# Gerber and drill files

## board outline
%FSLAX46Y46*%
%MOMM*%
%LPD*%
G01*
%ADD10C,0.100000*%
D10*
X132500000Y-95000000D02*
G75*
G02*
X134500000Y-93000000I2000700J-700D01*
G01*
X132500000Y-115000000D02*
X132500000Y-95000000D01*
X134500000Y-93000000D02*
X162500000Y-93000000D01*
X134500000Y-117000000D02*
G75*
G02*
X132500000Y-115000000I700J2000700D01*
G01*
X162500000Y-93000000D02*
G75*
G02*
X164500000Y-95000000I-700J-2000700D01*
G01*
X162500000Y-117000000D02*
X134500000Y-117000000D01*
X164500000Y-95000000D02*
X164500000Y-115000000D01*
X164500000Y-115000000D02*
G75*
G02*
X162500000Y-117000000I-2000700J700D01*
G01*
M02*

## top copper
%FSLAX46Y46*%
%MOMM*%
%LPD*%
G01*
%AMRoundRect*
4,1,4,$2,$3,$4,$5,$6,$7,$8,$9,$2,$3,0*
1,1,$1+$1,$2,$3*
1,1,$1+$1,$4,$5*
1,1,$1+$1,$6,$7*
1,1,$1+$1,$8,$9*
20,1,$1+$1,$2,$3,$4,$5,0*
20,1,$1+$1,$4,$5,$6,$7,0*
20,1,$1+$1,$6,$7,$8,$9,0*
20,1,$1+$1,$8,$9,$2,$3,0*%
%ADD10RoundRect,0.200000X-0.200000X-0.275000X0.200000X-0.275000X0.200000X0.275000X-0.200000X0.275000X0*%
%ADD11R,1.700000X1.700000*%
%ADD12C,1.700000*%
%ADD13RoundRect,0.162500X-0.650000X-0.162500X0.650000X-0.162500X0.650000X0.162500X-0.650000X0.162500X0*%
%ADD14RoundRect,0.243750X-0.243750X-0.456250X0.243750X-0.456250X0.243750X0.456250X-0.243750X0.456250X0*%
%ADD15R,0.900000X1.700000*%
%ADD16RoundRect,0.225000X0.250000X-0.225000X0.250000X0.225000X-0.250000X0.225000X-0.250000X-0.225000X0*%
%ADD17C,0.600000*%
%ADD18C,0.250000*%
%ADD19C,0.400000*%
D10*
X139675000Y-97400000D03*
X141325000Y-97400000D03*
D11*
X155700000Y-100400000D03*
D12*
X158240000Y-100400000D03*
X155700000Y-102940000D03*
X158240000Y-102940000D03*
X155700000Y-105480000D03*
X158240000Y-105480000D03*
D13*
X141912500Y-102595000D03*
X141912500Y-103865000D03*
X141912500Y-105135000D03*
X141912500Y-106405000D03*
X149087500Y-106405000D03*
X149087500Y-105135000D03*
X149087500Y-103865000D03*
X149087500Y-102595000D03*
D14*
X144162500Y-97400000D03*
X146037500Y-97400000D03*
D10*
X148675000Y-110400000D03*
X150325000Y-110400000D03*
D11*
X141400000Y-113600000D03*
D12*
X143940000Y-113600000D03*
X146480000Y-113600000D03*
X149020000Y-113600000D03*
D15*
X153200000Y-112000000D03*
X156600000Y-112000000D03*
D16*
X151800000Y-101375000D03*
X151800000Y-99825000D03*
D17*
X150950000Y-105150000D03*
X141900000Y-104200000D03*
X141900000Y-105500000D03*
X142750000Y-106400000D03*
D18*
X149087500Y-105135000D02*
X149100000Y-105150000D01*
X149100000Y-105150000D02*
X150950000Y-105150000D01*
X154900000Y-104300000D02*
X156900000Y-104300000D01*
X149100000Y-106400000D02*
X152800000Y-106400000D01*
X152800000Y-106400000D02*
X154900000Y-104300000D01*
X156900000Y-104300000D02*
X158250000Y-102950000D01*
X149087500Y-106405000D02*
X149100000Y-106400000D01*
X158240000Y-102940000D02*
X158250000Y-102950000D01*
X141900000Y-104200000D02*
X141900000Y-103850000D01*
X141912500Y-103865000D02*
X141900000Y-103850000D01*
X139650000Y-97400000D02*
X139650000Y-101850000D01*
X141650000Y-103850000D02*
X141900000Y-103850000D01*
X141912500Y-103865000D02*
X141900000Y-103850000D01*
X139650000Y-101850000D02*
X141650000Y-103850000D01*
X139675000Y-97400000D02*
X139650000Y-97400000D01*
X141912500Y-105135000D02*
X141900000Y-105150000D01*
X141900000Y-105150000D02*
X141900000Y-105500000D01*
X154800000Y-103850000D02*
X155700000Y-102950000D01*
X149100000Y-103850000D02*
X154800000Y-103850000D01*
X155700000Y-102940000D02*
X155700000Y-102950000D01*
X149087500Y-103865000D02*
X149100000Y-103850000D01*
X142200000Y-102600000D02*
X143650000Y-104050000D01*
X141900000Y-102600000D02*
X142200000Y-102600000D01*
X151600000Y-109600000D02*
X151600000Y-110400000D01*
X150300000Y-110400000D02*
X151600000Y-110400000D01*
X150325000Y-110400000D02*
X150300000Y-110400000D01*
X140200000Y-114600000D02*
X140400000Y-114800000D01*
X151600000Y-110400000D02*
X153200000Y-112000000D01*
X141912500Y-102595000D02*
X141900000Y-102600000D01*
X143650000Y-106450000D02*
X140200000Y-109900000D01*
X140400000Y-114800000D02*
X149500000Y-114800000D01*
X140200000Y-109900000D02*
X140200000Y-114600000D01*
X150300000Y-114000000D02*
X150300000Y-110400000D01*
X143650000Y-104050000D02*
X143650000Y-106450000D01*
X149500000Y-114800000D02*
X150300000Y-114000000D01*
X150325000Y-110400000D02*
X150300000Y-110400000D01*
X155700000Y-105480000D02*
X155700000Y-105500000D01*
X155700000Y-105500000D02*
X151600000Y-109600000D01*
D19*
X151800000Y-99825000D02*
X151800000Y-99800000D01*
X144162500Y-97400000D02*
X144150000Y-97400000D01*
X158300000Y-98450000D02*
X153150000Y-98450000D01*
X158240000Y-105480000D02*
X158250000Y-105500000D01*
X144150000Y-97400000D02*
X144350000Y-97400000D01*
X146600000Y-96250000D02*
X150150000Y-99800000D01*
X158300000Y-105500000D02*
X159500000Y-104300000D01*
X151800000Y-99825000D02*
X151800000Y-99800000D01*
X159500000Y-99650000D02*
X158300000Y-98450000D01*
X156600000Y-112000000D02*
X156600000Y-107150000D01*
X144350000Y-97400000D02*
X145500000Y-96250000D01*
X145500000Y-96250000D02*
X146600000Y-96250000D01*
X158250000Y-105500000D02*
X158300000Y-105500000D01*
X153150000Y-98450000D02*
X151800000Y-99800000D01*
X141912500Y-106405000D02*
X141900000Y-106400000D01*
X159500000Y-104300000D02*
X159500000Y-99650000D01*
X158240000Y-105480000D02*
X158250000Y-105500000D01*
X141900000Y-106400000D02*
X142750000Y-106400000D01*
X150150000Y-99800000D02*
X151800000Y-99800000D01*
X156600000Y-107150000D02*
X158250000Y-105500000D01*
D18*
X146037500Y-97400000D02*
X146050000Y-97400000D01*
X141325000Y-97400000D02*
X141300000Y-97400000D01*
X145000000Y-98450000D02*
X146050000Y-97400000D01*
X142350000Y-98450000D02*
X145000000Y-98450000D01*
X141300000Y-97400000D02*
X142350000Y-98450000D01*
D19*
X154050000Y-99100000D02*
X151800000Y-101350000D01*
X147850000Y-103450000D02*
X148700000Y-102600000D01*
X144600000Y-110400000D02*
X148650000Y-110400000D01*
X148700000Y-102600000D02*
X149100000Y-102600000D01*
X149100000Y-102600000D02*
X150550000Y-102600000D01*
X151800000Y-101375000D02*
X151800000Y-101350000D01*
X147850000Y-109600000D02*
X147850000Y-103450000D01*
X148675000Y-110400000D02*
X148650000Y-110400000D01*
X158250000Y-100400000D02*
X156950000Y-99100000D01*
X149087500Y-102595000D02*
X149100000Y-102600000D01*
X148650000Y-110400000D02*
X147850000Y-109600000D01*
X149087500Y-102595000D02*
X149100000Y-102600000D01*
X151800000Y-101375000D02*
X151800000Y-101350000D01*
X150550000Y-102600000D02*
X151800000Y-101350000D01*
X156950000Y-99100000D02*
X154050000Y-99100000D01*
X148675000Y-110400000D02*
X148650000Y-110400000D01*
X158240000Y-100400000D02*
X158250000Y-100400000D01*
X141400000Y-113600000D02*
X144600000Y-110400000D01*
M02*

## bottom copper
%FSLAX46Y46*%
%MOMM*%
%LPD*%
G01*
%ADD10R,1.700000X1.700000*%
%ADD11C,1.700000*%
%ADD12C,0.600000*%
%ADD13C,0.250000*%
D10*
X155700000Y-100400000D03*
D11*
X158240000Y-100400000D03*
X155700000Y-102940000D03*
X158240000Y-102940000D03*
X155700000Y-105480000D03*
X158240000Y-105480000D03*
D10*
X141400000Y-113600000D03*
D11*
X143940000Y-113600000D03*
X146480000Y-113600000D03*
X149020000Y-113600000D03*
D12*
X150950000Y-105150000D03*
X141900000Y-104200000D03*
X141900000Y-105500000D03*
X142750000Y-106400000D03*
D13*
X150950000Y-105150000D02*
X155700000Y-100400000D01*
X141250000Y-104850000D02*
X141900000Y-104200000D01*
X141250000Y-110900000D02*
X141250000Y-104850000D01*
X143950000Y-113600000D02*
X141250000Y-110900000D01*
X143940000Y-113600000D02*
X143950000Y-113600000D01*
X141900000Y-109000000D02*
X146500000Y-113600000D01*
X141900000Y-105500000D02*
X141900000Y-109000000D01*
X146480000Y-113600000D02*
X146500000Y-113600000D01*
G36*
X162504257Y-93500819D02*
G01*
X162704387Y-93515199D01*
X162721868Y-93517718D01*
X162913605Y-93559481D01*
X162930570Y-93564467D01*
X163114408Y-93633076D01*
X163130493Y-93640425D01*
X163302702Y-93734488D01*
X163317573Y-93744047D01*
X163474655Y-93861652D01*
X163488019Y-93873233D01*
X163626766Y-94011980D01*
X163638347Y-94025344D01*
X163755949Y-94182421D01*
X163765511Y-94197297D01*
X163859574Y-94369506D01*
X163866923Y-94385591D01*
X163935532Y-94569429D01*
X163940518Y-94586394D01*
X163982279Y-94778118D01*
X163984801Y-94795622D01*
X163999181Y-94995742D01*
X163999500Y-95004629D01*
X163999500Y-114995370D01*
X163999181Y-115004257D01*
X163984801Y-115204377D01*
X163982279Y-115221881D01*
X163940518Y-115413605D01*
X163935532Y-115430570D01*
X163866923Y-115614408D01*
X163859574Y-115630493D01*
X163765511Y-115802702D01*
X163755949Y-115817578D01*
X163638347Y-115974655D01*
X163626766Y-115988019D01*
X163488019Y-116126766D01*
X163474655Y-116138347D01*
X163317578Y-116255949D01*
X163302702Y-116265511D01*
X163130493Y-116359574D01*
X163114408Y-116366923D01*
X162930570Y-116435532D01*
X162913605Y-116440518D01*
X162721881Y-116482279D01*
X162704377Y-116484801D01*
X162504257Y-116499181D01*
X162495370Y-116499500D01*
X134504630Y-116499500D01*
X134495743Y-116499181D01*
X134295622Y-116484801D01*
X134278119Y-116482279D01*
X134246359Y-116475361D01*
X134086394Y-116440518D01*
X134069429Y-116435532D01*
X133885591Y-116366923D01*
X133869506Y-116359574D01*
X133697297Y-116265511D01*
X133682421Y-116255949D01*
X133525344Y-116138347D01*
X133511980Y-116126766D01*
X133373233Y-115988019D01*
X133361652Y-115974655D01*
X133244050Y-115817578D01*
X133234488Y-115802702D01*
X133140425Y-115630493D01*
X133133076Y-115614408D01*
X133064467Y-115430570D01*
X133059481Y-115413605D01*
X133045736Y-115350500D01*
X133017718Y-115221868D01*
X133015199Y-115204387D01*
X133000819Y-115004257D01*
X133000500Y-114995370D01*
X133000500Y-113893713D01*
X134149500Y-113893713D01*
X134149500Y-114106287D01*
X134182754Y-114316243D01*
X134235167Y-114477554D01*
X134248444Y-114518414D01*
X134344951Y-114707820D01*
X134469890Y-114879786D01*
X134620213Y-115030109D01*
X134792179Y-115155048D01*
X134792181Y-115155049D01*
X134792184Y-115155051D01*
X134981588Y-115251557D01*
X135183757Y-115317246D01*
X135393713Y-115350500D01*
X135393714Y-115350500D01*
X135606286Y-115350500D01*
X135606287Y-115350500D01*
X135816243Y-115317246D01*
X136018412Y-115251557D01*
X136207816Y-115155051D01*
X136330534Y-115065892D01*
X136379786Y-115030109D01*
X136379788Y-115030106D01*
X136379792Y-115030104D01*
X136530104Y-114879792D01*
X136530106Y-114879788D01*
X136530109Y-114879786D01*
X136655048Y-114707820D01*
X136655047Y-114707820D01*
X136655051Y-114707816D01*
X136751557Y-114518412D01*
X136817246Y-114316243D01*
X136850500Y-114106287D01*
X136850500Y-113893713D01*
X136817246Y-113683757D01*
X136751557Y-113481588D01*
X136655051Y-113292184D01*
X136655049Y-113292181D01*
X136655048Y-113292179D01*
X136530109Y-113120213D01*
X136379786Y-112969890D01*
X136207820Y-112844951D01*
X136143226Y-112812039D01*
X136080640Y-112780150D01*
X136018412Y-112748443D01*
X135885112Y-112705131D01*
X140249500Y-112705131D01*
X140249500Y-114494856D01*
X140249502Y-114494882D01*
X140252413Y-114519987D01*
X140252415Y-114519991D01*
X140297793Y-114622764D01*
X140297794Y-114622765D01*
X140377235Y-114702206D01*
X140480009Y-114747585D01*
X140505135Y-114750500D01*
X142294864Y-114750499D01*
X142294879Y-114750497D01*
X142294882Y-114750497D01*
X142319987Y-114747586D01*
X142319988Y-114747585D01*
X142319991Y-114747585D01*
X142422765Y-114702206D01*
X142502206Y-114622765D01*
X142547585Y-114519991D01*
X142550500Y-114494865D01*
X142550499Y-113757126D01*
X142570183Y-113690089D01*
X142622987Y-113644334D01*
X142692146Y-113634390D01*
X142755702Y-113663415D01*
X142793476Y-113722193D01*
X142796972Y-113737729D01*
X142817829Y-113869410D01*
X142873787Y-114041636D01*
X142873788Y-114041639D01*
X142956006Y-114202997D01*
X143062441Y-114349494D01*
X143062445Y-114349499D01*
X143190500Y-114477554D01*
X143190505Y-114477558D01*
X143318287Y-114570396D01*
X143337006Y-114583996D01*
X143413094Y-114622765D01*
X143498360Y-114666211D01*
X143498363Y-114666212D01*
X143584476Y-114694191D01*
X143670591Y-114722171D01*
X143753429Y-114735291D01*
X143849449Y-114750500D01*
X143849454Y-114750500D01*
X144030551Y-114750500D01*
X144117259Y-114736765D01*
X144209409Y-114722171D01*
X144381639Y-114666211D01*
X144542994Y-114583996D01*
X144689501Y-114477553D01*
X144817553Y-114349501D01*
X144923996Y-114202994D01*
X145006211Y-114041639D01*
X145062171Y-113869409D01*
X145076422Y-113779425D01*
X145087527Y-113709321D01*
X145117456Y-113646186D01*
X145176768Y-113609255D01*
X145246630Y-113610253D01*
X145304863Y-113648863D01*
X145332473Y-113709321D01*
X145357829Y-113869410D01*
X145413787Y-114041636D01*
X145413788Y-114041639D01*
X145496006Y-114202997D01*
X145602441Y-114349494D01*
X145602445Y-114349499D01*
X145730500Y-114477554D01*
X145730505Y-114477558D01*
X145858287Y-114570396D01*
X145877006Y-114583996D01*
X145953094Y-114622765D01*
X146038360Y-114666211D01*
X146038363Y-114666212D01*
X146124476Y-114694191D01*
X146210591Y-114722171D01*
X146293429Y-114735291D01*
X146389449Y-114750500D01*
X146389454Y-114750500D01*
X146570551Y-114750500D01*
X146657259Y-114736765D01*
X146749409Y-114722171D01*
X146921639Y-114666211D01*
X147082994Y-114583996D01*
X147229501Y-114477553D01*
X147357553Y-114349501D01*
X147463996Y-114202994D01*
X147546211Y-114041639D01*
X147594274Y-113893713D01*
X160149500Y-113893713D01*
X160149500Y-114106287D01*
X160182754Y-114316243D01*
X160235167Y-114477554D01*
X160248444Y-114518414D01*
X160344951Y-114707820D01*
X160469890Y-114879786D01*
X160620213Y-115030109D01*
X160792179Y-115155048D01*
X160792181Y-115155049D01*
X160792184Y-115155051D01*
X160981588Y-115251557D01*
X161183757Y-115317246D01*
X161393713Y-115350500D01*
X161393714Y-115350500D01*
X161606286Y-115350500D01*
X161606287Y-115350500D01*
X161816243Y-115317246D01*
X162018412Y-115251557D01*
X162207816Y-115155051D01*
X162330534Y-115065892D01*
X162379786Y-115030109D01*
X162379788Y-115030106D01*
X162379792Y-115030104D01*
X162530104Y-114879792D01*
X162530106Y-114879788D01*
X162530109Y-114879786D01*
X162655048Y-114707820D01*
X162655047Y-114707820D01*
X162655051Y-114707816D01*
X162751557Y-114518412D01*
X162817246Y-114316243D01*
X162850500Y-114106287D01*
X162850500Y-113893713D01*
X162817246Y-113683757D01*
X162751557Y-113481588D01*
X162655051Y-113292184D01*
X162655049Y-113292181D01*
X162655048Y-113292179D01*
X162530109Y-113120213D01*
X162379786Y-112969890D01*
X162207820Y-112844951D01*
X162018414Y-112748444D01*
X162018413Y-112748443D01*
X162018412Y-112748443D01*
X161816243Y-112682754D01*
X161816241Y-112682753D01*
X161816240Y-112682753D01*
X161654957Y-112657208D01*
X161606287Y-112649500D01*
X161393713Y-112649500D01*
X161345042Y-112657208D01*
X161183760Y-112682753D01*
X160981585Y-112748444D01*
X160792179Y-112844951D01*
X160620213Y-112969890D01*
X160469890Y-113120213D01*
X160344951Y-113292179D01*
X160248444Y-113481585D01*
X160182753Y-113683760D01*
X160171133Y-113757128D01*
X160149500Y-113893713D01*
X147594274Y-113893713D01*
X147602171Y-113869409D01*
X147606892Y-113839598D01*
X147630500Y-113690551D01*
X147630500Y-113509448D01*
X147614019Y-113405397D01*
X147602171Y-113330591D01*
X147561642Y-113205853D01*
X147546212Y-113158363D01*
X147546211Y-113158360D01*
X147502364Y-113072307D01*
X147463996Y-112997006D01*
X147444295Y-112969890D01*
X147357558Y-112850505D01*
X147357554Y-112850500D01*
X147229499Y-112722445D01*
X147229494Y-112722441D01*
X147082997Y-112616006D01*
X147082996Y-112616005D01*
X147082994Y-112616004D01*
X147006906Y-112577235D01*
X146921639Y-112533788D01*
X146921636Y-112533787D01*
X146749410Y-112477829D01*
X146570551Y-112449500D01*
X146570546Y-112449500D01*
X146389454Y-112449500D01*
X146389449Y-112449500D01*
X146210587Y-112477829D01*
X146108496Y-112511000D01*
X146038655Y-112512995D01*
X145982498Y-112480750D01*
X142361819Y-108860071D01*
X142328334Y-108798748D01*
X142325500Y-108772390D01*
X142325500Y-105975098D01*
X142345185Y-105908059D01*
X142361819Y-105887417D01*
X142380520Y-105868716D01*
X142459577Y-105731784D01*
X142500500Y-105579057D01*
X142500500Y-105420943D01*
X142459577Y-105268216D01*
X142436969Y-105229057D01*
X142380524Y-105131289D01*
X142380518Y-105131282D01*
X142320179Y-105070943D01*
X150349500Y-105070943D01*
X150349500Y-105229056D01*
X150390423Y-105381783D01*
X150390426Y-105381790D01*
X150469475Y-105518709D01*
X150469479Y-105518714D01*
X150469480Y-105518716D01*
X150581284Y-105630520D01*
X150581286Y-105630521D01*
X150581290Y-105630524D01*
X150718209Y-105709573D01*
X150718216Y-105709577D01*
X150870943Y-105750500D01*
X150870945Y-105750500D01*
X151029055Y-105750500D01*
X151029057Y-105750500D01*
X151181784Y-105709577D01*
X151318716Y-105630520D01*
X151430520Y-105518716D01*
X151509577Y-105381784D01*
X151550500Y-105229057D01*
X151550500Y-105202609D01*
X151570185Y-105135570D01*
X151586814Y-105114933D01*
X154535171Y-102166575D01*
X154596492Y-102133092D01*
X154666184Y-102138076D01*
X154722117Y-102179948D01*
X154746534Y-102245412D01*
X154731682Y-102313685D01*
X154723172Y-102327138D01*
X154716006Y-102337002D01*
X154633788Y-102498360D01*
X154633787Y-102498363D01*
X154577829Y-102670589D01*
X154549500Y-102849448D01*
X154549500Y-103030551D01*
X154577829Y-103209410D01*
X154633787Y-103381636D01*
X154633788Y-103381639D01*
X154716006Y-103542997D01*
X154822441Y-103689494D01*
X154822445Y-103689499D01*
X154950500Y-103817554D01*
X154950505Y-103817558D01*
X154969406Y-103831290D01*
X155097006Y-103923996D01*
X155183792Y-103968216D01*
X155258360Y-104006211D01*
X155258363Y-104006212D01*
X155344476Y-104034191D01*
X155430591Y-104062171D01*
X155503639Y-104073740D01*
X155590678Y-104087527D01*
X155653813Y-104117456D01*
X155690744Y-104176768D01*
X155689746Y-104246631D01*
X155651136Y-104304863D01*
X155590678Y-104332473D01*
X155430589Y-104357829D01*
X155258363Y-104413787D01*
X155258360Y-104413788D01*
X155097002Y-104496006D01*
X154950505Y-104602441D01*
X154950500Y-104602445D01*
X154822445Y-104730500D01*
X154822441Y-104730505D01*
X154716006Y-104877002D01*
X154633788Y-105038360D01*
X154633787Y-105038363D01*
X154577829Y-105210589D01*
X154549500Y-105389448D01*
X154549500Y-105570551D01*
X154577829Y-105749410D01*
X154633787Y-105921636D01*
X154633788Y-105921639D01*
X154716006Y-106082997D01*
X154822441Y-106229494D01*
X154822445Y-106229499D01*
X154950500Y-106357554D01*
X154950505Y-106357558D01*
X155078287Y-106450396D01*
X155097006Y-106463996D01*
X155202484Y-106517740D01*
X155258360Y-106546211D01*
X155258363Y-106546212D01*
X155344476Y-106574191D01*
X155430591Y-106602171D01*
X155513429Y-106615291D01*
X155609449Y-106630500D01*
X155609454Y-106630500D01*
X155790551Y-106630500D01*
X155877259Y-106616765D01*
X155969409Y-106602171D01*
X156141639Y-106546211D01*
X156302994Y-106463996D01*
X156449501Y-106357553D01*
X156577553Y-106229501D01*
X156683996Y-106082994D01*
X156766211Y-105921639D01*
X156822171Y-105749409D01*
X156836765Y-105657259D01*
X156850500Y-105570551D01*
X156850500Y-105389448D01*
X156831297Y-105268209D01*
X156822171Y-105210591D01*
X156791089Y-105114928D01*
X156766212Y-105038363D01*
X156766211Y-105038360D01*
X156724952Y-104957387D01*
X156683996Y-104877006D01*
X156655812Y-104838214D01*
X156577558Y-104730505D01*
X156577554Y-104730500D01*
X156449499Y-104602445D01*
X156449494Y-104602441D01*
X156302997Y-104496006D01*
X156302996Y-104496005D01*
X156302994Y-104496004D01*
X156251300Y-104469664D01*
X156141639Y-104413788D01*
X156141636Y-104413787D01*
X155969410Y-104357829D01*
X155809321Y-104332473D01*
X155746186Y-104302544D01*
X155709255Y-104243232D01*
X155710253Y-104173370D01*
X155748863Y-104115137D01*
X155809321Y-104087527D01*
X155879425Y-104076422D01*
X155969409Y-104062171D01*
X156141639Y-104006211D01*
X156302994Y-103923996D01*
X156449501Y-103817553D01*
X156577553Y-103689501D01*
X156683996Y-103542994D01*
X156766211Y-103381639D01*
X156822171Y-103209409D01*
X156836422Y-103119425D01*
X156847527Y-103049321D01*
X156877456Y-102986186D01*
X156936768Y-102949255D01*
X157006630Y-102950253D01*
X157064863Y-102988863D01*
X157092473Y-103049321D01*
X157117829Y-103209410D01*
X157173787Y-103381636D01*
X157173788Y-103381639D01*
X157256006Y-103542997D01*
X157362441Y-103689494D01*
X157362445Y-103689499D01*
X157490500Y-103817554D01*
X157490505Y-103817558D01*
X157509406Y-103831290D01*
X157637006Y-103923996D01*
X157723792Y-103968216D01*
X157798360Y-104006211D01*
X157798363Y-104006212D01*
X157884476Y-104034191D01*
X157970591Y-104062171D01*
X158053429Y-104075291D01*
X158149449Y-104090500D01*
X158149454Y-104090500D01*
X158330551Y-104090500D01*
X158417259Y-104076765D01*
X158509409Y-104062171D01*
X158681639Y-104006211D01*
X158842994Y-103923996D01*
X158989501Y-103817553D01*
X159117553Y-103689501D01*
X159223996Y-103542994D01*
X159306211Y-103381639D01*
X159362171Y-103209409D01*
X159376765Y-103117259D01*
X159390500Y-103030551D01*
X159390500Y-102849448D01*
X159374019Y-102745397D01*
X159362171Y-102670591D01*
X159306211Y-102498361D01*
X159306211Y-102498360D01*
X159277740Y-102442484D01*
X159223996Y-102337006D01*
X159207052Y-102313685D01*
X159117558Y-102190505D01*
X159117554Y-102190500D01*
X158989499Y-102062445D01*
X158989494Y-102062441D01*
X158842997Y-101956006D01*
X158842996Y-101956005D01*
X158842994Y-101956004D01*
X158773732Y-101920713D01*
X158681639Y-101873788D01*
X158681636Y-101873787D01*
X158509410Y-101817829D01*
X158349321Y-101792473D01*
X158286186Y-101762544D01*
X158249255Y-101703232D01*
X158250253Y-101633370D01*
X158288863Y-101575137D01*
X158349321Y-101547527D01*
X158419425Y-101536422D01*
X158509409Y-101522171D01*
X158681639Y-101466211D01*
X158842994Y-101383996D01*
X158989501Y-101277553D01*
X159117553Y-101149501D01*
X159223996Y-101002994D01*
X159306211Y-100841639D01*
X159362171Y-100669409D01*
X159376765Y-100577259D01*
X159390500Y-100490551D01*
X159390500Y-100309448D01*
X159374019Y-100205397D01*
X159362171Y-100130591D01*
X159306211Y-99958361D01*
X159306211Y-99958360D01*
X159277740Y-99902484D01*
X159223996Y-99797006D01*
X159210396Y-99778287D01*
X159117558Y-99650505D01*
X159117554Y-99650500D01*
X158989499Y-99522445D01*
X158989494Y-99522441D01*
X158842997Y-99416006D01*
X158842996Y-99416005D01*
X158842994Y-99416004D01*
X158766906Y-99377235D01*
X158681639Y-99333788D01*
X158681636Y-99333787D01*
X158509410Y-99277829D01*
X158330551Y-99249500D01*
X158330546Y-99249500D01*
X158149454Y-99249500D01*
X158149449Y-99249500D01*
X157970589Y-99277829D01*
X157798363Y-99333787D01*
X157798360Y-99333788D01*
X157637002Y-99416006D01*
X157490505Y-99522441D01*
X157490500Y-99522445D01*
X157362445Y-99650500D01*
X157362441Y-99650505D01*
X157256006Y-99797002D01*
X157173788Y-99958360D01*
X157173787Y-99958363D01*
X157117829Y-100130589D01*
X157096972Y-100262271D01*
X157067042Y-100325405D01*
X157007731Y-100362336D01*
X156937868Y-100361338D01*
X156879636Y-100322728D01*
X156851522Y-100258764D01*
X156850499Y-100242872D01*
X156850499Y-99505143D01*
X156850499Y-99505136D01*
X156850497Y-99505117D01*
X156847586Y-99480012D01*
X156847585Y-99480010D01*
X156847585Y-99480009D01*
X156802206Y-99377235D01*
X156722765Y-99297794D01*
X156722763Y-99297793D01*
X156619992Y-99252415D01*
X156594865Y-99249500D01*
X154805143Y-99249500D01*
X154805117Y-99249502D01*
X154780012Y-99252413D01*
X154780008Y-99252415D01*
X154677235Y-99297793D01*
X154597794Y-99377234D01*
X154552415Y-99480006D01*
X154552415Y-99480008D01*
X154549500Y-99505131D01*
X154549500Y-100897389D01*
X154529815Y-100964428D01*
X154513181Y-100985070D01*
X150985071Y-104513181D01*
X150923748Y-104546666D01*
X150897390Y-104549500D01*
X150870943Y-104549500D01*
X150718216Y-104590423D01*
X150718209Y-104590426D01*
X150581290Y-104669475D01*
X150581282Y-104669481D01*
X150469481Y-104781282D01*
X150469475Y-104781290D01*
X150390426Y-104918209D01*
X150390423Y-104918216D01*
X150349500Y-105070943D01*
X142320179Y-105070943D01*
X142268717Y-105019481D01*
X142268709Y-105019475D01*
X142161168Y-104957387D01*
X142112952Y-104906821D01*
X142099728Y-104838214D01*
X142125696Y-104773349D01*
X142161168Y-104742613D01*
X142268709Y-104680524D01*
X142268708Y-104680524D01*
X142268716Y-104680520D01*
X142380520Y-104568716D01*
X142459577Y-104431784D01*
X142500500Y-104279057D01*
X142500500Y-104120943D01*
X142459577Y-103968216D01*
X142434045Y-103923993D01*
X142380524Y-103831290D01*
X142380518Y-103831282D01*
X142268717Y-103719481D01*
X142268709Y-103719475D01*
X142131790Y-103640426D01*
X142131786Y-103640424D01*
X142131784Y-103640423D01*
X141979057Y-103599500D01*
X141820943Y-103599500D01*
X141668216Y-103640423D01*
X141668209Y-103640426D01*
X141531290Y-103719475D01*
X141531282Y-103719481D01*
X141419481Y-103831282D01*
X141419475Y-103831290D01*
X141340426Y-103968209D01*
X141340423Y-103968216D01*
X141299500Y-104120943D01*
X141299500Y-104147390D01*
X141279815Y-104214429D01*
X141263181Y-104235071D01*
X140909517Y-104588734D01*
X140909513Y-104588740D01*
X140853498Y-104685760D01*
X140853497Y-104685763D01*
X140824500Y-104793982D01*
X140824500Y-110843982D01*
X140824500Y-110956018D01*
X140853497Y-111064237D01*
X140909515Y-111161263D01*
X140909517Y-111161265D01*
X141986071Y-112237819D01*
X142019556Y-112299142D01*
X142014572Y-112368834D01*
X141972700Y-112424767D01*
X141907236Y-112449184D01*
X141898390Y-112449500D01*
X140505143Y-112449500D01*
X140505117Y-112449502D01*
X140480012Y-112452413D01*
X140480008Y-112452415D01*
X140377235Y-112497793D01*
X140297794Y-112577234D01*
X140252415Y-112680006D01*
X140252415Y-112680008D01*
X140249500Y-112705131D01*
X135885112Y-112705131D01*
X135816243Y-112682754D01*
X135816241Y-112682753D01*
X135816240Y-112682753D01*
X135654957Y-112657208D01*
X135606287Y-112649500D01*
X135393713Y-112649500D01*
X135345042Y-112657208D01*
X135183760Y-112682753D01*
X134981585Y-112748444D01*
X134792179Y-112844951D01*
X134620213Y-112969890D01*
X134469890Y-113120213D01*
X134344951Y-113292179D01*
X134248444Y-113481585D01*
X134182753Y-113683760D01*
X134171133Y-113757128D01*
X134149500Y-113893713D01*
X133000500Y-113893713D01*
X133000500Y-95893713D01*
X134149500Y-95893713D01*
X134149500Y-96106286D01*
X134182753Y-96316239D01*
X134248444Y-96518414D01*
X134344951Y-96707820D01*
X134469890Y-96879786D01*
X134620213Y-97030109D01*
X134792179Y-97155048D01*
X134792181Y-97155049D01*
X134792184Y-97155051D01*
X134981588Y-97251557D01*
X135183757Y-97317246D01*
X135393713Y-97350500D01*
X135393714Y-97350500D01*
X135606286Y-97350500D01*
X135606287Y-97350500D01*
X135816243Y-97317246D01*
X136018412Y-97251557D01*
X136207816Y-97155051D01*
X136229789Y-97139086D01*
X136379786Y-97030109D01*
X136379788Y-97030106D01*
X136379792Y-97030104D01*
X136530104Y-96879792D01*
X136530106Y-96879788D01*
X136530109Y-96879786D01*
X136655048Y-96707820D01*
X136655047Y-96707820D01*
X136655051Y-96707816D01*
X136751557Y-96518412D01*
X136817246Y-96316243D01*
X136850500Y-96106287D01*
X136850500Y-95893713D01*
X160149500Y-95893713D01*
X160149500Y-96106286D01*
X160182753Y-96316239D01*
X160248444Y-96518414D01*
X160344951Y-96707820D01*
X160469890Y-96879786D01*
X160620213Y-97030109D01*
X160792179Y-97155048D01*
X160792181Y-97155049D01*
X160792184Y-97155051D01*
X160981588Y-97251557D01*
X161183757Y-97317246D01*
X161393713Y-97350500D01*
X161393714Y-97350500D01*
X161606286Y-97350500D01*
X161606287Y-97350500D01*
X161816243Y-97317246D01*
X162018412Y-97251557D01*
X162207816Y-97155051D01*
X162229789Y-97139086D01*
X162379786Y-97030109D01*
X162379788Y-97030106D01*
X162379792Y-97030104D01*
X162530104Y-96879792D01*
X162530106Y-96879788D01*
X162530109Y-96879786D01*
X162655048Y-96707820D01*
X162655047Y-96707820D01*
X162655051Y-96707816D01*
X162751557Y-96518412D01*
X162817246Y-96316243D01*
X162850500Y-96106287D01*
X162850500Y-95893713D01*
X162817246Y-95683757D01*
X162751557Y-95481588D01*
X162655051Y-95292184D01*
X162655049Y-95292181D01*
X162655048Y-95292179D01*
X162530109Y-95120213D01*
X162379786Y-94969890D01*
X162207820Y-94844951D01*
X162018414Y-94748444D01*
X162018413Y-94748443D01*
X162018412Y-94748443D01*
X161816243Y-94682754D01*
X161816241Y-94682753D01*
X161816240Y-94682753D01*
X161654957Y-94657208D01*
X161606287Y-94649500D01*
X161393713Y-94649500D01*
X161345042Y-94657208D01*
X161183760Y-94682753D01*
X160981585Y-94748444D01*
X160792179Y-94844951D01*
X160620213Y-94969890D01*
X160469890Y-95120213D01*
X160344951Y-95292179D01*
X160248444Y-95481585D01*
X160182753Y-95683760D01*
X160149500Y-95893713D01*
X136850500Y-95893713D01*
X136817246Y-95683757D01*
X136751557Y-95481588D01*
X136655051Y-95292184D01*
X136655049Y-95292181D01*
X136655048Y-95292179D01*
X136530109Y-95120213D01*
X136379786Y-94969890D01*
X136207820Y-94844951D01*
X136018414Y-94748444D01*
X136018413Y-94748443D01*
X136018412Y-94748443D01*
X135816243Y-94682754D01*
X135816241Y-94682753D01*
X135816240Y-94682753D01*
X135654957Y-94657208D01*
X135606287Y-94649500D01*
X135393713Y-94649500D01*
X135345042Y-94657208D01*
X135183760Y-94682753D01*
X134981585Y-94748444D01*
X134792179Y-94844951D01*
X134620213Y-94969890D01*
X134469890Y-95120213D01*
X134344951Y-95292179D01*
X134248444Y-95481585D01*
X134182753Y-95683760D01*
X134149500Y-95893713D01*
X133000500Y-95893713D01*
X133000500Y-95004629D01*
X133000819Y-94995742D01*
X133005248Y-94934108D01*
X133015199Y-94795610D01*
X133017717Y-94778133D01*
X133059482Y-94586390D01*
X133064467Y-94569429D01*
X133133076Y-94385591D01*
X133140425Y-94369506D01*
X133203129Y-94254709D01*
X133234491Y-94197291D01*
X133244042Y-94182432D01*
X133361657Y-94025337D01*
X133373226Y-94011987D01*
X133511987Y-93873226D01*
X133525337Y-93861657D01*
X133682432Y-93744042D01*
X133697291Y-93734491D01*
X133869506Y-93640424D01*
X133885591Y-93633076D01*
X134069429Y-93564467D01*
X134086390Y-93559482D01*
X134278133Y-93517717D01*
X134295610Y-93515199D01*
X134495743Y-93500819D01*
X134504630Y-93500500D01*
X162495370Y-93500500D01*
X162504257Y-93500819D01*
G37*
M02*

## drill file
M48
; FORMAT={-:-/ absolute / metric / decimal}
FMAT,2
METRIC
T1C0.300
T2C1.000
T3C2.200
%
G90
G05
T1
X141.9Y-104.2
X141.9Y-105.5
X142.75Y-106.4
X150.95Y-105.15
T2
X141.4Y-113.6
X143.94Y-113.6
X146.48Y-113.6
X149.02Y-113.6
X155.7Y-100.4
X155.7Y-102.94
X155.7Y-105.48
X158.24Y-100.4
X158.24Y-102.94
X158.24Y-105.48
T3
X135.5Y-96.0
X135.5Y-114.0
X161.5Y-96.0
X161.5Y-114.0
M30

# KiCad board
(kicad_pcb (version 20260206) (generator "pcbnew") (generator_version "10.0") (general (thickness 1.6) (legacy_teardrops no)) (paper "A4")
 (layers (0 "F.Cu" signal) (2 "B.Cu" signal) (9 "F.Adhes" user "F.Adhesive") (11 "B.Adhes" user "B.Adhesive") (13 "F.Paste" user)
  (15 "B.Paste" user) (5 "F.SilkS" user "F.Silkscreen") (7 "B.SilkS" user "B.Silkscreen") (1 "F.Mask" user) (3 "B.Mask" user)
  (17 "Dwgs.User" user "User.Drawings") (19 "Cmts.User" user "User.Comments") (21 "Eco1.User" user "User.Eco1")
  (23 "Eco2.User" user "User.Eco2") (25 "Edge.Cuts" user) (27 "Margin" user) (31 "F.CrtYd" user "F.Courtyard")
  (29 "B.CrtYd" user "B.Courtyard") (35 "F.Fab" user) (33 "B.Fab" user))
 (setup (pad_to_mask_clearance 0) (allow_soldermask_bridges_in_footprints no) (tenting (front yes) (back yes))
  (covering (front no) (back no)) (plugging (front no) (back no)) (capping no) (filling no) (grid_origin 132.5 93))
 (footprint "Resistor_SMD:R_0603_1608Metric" (layer "F.Cu") (at 140.5 97.4)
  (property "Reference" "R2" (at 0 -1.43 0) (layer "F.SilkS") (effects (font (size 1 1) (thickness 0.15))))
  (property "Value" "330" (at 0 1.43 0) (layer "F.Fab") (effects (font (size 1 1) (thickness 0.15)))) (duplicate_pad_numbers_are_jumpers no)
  (pad "1" smd roundrect (at -0.825 0) (size 0.8 0.95) (layers "F.Cu" "F.Mask" "F.Paste") (roundrect_rratio 0.25) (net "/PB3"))
  (pad "2" smd roundrect (at 0.825 0) (size 0.8 0.95) (layers "F.Cu" "F.Mask" "F.Paste") (roundrect_rratio 0.25) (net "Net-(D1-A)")))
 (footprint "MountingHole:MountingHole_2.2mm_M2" (layer "F.Cu") (at 161.5 114)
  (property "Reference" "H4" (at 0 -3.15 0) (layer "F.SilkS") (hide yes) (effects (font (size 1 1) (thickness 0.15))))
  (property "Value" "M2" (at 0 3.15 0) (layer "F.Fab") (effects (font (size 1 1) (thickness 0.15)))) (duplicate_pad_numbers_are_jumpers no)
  (pad "" np_thru_hole circle (at 0 0) (size 2.2 2.2) (drill 2.2) (layers "*.Cu" "*.Mask")))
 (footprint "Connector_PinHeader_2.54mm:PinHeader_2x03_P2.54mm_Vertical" (layer "F.Cu") (at 155.7 100.4)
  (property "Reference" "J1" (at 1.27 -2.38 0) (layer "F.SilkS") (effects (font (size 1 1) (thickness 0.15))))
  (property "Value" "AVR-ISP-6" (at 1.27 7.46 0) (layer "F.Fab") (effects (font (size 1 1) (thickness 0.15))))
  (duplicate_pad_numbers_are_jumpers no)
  (pad "1" thru_hole rect (at 0 0) (size 1.7 1.7) (drill 1) (layers "*.Cu" "*.Mask") (remove_unused_layers no) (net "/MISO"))
  (pad "2" thru_hole circle (at 2.54 0) (size 1.7 1.7) (drill 1) (layers "*.Cu" "*.Mask") (remove_unused_layers no) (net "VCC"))
  (pad "3" thru_hole circle (at 0 2.54) (size 1.7 1.7) (drill 1) (layers "*.Cu" "*.Mask") (remove_unused_layers no) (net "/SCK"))
  (pad "4" thru_hole circle (at 2.54 2.54) (size 1.7 1.7) (drill 1) (layers "*.Cu" "*.Mask") (remove_unused_layers no) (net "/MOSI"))
  (pad "5" thru_hole circle (at 0 5.08) (size 1.7 1.7) (drill 1) (layers "*.Cu" "*.Mask") (remove_unused_layers no) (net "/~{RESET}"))
  (pad "6" thru_hole circle (at 2.54 5.08) (size 1.7 1.7) (drill 1) (layers "*.Cu" "*.Mask") (remove_unused_layers no) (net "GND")))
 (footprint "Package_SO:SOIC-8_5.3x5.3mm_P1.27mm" (layer "F.Cu") (at 145.5 104.5)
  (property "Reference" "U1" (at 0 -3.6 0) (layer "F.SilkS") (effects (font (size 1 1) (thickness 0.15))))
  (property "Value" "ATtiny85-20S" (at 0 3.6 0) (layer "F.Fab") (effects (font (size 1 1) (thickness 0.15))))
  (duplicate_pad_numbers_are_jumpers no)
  (pad "1" smd roundrect (at -3.5875 -1.905) (size 1.625 0.65) (layers "F.Cu" "F.Mask" "F.Paste") (roundrect_rratio 0.25) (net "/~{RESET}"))
  (pad "2" smd roundrect (at -3.5875 -0.635) (size 1.625 0.65) (layers "F.Cu" "F.Mask" "F.Paste") (roundrect_rratio 0.25) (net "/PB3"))
  (pad "3" smd roundrect (at -3.5875 0.635) (size 1.625 0.65) (layers "F.Cu" "F.Mask" "F.Paste") (roundrect_rratio 0.25) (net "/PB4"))
  (pad "4" smd roundrect (at -3.5875 1.905) (size 1.625 0.65) (layers "F.Cu" "F.Mask" "F.Paste") (roundrect_rratio 0.25) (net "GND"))
  (pad "5" smd roundrect (at 3.5875 1.905) (size 1.625 0.65) (layers "F.Cu" "F.Mask" "F.Paste") (roundrect_rratio 0.25) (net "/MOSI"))
  (pad "6" smd roundrect (at 3.5875 0.635) (size 1.625 0.65) (layers "F.Cu" "F.Mask" "F.Paste") (roundrect_rratio 0.25) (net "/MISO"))
  (pad "7" smd roundrect (at 3.5875 -0.635) (size 1.625 0.65) (layers "F.Cu" "F.Mask" "F.Paste") (roundrect_rratio 0.25) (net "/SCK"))
  (pad "8" smd roundrect (at 3.5875 -1.905) (size 1.625 0.65) (layers "F.Cu" "F.Mask" "F.Paste") (roundrect_rratio 0.25) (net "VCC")))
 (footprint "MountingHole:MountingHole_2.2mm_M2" (layer "F.Cu") (at 161.5 96)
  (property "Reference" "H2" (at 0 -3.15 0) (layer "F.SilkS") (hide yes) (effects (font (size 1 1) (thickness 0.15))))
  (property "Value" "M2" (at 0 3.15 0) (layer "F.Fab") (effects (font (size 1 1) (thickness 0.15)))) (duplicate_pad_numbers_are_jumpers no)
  (pad "" np_thru_hole circle (at 0 0) (size 2.2 2.2) (drill 2.2) (layers "*.Cu" "*.Mask")))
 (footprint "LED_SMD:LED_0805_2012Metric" (layer "F.Cu") (at 145.1 97.4)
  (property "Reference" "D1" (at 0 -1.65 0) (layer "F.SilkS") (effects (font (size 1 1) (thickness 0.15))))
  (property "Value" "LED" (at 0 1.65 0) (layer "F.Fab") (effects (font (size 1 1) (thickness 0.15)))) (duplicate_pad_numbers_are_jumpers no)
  (pad "1" smd roundrect (at -0.9375 0) (size 0.975 1.4) (layers "F.Cu" "F.Mask" "F.Paste") (roundrect_rratio 0.25) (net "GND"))
  (pad "2" smd roundrect (at 0.9375 0) (size 0.975 1.4) (layers "F.Cu" "F.Mask" "F.Paste") (roundrect_rratio 0.25) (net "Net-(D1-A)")))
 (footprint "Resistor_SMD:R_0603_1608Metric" (layer "F.Cu") (at 149.5 110.4)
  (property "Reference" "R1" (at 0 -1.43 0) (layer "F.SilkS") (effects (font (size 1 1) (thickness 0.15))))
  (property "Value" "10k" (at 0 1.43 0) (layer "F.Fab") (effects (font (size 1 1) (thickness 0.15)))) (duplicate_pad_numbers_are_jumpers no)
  (pad "1" smd roundrect (at -0.825 0) (size 0.8 0.95) (layers "F.Cu" "F.Mask" "F.Paste") (roundrect_rratio 0.25) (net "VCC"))
  (pad "2" smd roundrect (at 0.825 0) (size 0.8 0.95) (layers "F.Cu" "F.Mask" "F.Paste") (roundrect_rratio 0.25) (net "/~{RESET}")))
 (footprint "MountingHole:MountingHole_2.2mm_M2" (layer "F.Cu") (at 135.5 96)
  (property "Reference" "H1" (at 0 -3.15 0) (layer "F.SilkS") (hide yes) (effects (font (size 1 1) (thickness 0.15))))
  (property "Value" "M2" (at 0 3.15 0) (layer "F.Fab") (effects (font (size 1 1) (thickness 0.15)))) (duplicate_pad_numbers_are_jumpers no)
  (pad "" np_thru_hole circle (at 0 0) (size 2.2 2.2) (drill 2.2) (layers "*.Cu" "*.Mask")))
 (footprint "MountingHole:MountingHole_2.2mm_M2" (layer "F.Cu") (at 135.5 114)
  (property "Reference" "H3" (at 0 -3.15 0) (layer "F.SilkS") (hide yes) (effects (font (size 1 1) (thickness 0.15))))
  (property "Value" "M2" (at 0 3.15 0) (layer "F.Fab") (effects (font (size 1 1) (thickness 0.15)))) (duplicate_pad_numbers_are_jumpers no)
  (pad "" np_thru_hole circle (at 0 0) (size 2.2 2.2) (drill 2.2) (layers "*.Cu" "*.Mask")))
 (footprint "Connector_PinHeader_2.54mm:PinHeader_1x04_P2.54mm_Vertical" (layer "F.Cu") (at 141.4 113.6 90)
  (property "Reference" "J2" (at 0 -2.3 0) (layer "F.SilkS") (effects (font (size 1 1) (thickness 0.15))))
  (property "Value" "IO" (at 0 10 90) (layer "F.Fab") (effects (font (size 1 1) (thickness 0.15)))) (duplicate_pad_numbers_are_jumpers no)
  (pad "1" thru_hole rect (at 0 0 90) (size 1.7 1.7) (drill 1) (layers "*.Cu" "*.Mask") (remove_unused_layers no) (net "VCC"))
  (pad "2" thru_hole circle (at 0 2.54 90) (size 1.7 1.7) (drill 1) (layers "*.Cu" "*.Mask") (remove_unused_layers no) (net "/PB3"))
  (pad "3" thru_hole circle (at 0 5.08 90) (size 1.7 1.7) (drill 1) (layers "*.Cu" "*.Mask") (remove_unused_layers no) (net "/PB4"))
  (pad "4" thru_hole circle (at 0 7.62 90) (size 1.7 1.7) (drill 1) (layers "*.Cu" "*.Mask") (remove_unused_layers no) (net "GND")))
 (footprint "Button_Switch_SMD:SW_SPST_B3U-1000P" (layer "F.Cu") (at 154.9 112)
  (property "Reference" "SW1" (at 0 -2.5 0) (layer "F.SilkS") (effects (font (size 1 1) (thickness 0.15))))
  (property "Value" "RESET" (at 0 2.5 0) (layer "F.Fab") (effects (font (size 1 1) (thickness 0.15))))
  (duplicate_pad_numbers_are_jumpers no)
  (pad "1" smd rect (at -1.7 0) (size 0.9 1.7) (layers "F.Cu" "F.Mask" "F.Paste") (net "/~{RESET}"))
  (pad "2" smd rect (at 1.7 0) (size 0.9 1.7) (layers "F.Cu" "F.Mask" "F.Paste") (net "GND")))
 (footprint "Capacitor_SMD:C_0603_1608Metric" (layer "F.Cu") (at 151.8 100.6 90)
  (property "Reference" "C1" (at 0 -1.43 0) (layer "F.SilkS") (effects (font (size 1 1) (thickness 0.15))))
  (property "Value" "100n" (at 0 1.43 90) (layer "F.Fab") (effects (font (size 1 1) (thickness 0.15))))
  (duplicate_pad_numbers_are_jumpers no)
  (pad "1" smd roundrect (at -0.775 0 90) (size 0.9 0.95) (layers "F.Cu" "F.Mask" "F.Paste") (roundrect_rratio 0.25) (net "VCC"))
  (pad "2" smd roundrect (at 0.775 0 90) (size 0.9 0.95) (layers "F.Cu" "F.Mask" "F.Paste") (roundrect_rratio 0.25) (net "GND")))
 (gr_arc (start 132.5 95) (mid 133.086 93.586) (end 134.5 93) (stroke (width 0.1) (type default)) (layer "Edge.Cuts"))
 (gr_line (start 132.5 115) (end 132.5 95) (stroke (width 0.1) (type default)) (layer "Edge.Cuts"))
 (gr_line (start 134.5 93) (end 162.5 93) (stroke (width 0.1) (type default)) (layer "Edge.Cuts"))
 (gr_arc (start 134.5 117) (mid 133.086 116.414) (end 132.5 115) (stroke (width 0.1) (type default)) (layer "Edge.Cuts"))
 (gr_arc (start 162.5 93) (mid 163.914 93.586) (end 164.5 95) (stroke (width 0.1) (type default)) (layer "Edge.Cuts"))
 (gr_line (start 162.5 117) (end 134.5 117) (stroke (width 0.1) (type default)) (layer "Edge.Cuts"))
 (gr_line (start 164.5 95) (end 164.5 115) (stroke (width 0.1) (type default)) (layer "Edge.Cuts"))
 (gr_arc (start 164.5 115) (mid 163.914 116.414) (end 162.5 117) (stroke (width 0.1) (type default)) (layer "Edge.Cuts"))
 (segment (start 149.0875 105.135) (end 149.1 105.15) (width 0.25) (layer "F.Cu") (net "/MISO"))
 (segment (start 149.1 105.15) (end 150.95 105.15) (width 0.25) (layer "F.Cu") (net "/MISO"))
 (via (at 150.95 105.15) (size 0.6) (drill 0.3) (layers "F.Cu" "B.Cu") (capping no) (covering (front no) (back no))
  (plugging (front no) (back no)) (filling no) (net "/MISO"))
 (segment (start 150.95 105.15) (end 155.7 100.4) (width 0.25) (layer "B.Cu") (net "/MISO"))
 (segment (start 154.9 104.3) (end 156.9 104.3) (width 0.25) (layer "F.Cu") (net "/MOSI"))
 (segment (start 149.1 106.4) (end 152.8 106.4) (width 0.25) (layer "F.Cu") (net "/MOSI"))
 (segment (start 152.8 106.4) (end 154.9 104.3) (width 0.25) (layer "F.Cu") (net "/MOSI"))
 (segment (start 156.9 104.3) (end 158.25 102.95) (width 0.25) (layer "F.Cu") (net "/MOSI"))
 (segment (start 149.0875 106.405) (end 149.1 106.4) (width 0.25) (layer "F.Cu") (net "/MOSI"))
 (segment (start 158.24 102.94) (end 158.25 102.95) (width 0.25) (layer "F.Cu") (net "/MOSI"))
 (segment (start 141.9 104.2) (end 141.9 103.85) (width 0.25) (layer "F.Cu") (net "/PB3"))
 (segment (start 141.9125 103.865) (end 141.9 103.85) (width 0.25) (layer "F.Cu") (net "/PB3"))
 (segment (start 139.65 97.4) (end 139.65 101.85) (width 0.25) (layer "F.Cu") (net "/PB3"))
 (segment (start 141.65 103.85) (end 141.9 103.85) (width 0.25) (layer "F.Cu") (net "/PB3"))
 (segment (start 141.9125 103.865) (end 141.9 103.85) (width 0.25) (layer "F.Cu") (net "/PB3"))
 (segment (start 139.65 101.85) (end 141.65 103.85) (width 0.25) (layer "F.Cu") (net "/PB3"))
 (segment (start 139.675 97.4) (end 139.65 97.4) (width 0.25) (layer "F.Cu") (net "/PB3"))
 (via (at 141.9 104.2) (size 0.6) (drill 0.3) (layers "F.Cu" "B.Cu") (capping no) (covering (front no) (back no))
  (plugging (front no) (back no)) (filling no) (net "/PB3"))
 (segment (start 141.25 104.85) (end 141.9 104.2) (width 0.25) (layer "B.Cu") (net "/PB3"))
 (segment (start 141.25 110.9) (end 141.25 104.85) (width 0.25) (layer "B.Cu") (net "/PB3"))
 (segment (start 143.95 113.6) (end 141.25 110.9) (width 0.25) (layer "B.Cu") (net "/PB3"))
 (segment (start 143.94 113.6) (end 143.95 113.6) (width 0.25) (layer "B.Cu") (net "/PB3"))
 (segment (start 141.9125 105.135) (end 141.9 105.15) (width 0.25) (layer "F.Cu") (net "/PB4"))
 (segment (start 141.9 105.15) (end 141.9 105.5) (width 0.25) (layer "F.Cu") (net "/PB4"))
 (via (at 141.9 105.5) (size 0.6) (drill 0.3) (layers "F.Cu" "B.Cu") (capping no) (covering (front no) (back no))
  (plugging (front no) (back no)) (filling no) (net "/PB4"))
 (segment (start 141.9 109) (end 146.5 113.6) (width 0.25) (layer "B.Cu") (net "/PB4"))
 (segment (start 141.9 105.5) (end 141.9 109) (width 0.25) (layer "B.Cu") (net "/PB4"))
 (segment (start 146.48 113.6) (end 146.5 113.6) (width 0.25) (layer "B.Cu") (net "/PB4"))
 (segment (start 154.8 103.85) (end 155.7 102.95) (width 0.25) (layer "F.Cu") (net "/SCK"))
 (segment (start 149.1 103.85) (end 154.8 103.85) (width 0.25) (layer "F.Cu") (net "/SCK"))
 (segment (start 155.7 102.94) (end 155.7 102.95) (width 0.25) (layer "F.Cu") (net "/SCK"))
 (segment (start 149.0875 103.865) (end 149.1 103.85) (width 0.25) (layer "F.Cu") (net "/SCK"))
 (segment (start 142.2 102.6) (end 143.65 104.05) (width 0.25) (layer "F.Cu") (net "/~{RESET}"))
 (segment (start 141.9 102.6) (end 142.2 102.6) (width 0.25) (layer "F.Cu") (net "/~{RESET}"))
 (segment (start 151.6 109.6) (end 151.6 110.4) (width 0.25) (layer "F.Cu") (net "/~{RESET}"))
 (segment (start 150.3 110.4) (end 151.6 110.4) (width 0.25) (layer "F.Cu") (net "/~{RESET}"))
 (segment (start 150.325 110.4) (end 150.3 110.4) (width 0.25) (layer "F.Cu") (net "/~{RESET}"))
 (segment (start 140.2 114.6) (end 140.4 114.8) (width 0.25) (layer "F.Cu") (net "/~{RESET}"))
 (segment (start 151.6 110.4) (end 153.2 112) (width 0.25) (layer "F.Cu") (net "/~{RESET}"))
 (segment (start 141.9125 102.595) (end 141.9 102.6) (width 0.25) (layer "F.Cu") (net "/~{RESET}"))
 (segment (start 143.65 106.45) (end 140.2 109.9) (width 0.25) (layer "F.Cu") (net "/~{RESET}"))
 (segment (start 140.4 114.8) (end 149.5 114.8) (width 0.25) (layer "F.Cu") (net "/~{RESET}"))
 (segment (start 140.2 109.9) (end 140.2 114.6) (width 0.25) (layer "F.Cu") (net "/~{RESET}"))
 (segment (start 150.3 114) (end 150.3 110.4) (width 0.25) (layer "F.Cu") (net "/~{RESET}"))
 (segment (start 143.65 104.05) (end 143.65 106.45) (width 0.25) (layer "F.Cu") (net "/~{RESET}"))
 (segment (start 149.5 114.8) (end 150.3 114) (width 0.25) (layer "F.Cu") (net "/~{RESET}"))
 (segment (start 150.325 110.4) (end 150.3 110.4) (width 0.25) (layer "F.Cu") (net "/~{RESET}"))
 (segment (start 155.7 105.48) (end 155.7 105.5) (width 0.25) (layer "F.Cu") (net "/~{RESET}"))
 (segment (start 155.7 105.5) (end 151.6 109.6) (width 0.25) (layer "F.Cu") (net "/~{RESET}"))
 (segment (start 151.8 99.825) (end 151.8 99.8) (width 0.4) (layer "F.Cu") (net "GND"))
 (segment (start 144.1625 97.4) (end 144.15 97.4) (width 0.4) (layer "F.Cu") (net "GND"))
 (segment (start 158.3 98.45) (end 153.15 98.45) (width 0.4) (layer "F.Cu") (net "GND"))
 (segment (start 158.24 105.48) (end 158.25 105.5) (width 0.4) (layer "F.Cu") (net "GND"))
 (segment (start 144.15 97.4) (end 144.35 97.4) (width 0.4) (layer "F.Cu") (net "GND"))
 (segment (start 146.6 96.25) (end 150.15 99.8) (width 0.4) (layer "F.Cu") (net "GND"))
 (segment (start 158.3 105.5) (end 159.5 104.3) (width 0.4) (layer "F.Cu") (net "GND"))
 (segment (start 151.8 99.825) (end 151.8 99.8) (width 0.4) (layer "F.Cu") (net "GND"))
 (segment (start 159.5 99.65) (end 158.3 98.45) (width 0.4) (layer "F.Cu") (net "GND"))
 (segment (start 156.6 112) (end 156.6 107.15) (width 0.4) (layer "F.Cu") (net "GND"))
 (segment (start 144.35 97.4) (end 145.5 96.25) (width 0.4) (layer "F.Cu") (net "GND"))
 (segment (start 145.5 96.25) (end 146.6 96.25) (width 0.4) (layer "F.Cu") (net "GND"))
 (segment (start 158.25 105.5) (end 158.3 105.5) (width 0.4) (layer "F.Cu") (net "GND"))
 (segment (start 153.15 98.45) (end 151.8 99.8) (width 0.4) (layer "F.Cu") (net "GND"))
 (segment (start 141.9125 106.405) (end 141.9 106.4) (width 0.4) (layer "F.Cu") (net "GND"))
 (segment (start 159.5 104.3) (end 159.5 99.65) (width 0.4) (layer "F.Cu") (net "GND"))
 (segment (start 158.24 105.48) (end 158.25 105.5) (width 0.4) (layer "F.Cu") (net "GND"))
 (segment (start 141.9 106.4) (end 142.75 106.4) (width 0.4) (layer "F.Cu") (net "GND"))
 (segment (start 150.15 99.8) (end 151.8 99.8) (width 0.4) (layer "F.Cu") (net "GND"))
 (segment (start 156.6 107.15) (end 158.25 105.5) (width 0.4) (layer "F.Cu") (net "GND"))
 (via (at 142.75 106.4) (size 0.6) (drill 0.3) (layers "F.Cu" "B.Cu") (capping no) (covering (front no) (back no))
  (plugging (front no) (back no)) (filling no) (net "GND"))
 (segment (start 146.0375 97.4) (end 146.05 97.4) (width 0.25) (layer "F.Cu") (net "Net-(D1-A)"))
 (segment (start 141.325 97.4) (end 141.3 97.4) (width 0.25) (layer "F.Cu") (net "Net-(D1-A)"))
 (segment (start 145 98.45) (end 146.05 97.4) (width 0.25) (layer "F.Cu") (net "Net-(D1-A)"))
 (segment (start 142.35 98.45) (end 145 98.45) (width 0.25) (layer "F.Cu") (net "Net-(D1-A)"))
 (segment (start 141.3 97.4) (end 142.35 98.45) (width 0.25) (layer "F.Cu") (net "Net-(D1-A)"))
 (segment (start 154.05 99.1) (end 151.8 101.35) (width 0.4) (layer "F.Cu") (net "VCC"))
 (segment (start 147.85 103.45) (end 148.7 102.6) (width 0.4) (layer "F.Cu") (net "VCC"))
 (segment (start 144.6 110.4) (end 148.65 110.4) (width 0.4) (layer "F.Cu") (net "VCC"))
 (segment (start 148.7 102.6) (end 149.1 102.6) (width 0.4) (layer "F.Cu") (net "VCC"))
 (segment (start 149.1 102.6) (end 150.55 102.6) (width 0.4) (layer "F.Cu") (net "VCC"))
 (segment (start 151.8 101.375) (end 151.8 101.35) (width 0.4) (layer "F.Cu") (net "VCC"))
 (segment (start 147.85 109.6) (end 147.85 103.45) (width 0.4) (layer "F.Cu") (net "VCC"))
 (segment (start 148.675 110.4) (end 148.65 110.4) (width 0.4) (layer "F.Cu") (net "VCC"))
 (segment (start 158.25 100.4) (end 156.95 99.1) (width 0.4) (layer "F.Cu") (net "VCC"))
 (segment (start 149.0875 102.595) (end 149.1 102.6) (width 0.4) (layer "F.Cu") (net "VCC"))
 (segment (start 148.65 110.4) (end 147.85 109.6) (width 0.4) (layer "F.Cu") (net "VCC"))
 (segment (start 149.0875 102.595) (end 149.1 102.6) (width 0.4) (layer "F.Cu") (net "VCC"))
 (segment (start 151.8 101.375) (end 151.8 101.35) (width 0.4) (layer "F.Cu") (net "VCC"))
 (segment (start 150.55 102.6) (end 151.8 101.35) (width 0.4) (layer "F.Cu") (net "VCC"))
 (segment (start 156.95 99.1) (end 154.05 99.1) (width 0.4) (layer "F.Cu") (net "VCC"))
 (segment (start 148.675 110.4) (end 148.65 110.4) (width 0.4) (layer "F.Cu") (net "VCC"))
 (segment (start 158.24 100.4) (end 158.25 100.4) (width 0.4) (layer "F.Cu") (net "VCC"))
 (segment (start 141.4 113.6) (end 144.6 110.4) (width 0.4) (layer "F.Cu") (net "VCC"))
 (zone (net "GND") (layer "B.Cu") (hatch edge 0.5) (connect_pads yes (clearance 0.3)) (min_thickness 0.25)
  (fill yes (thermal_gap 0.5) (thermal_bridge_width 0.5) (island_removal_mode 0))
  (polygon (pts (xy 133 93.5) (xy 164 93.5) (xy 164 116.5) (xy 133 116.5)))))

